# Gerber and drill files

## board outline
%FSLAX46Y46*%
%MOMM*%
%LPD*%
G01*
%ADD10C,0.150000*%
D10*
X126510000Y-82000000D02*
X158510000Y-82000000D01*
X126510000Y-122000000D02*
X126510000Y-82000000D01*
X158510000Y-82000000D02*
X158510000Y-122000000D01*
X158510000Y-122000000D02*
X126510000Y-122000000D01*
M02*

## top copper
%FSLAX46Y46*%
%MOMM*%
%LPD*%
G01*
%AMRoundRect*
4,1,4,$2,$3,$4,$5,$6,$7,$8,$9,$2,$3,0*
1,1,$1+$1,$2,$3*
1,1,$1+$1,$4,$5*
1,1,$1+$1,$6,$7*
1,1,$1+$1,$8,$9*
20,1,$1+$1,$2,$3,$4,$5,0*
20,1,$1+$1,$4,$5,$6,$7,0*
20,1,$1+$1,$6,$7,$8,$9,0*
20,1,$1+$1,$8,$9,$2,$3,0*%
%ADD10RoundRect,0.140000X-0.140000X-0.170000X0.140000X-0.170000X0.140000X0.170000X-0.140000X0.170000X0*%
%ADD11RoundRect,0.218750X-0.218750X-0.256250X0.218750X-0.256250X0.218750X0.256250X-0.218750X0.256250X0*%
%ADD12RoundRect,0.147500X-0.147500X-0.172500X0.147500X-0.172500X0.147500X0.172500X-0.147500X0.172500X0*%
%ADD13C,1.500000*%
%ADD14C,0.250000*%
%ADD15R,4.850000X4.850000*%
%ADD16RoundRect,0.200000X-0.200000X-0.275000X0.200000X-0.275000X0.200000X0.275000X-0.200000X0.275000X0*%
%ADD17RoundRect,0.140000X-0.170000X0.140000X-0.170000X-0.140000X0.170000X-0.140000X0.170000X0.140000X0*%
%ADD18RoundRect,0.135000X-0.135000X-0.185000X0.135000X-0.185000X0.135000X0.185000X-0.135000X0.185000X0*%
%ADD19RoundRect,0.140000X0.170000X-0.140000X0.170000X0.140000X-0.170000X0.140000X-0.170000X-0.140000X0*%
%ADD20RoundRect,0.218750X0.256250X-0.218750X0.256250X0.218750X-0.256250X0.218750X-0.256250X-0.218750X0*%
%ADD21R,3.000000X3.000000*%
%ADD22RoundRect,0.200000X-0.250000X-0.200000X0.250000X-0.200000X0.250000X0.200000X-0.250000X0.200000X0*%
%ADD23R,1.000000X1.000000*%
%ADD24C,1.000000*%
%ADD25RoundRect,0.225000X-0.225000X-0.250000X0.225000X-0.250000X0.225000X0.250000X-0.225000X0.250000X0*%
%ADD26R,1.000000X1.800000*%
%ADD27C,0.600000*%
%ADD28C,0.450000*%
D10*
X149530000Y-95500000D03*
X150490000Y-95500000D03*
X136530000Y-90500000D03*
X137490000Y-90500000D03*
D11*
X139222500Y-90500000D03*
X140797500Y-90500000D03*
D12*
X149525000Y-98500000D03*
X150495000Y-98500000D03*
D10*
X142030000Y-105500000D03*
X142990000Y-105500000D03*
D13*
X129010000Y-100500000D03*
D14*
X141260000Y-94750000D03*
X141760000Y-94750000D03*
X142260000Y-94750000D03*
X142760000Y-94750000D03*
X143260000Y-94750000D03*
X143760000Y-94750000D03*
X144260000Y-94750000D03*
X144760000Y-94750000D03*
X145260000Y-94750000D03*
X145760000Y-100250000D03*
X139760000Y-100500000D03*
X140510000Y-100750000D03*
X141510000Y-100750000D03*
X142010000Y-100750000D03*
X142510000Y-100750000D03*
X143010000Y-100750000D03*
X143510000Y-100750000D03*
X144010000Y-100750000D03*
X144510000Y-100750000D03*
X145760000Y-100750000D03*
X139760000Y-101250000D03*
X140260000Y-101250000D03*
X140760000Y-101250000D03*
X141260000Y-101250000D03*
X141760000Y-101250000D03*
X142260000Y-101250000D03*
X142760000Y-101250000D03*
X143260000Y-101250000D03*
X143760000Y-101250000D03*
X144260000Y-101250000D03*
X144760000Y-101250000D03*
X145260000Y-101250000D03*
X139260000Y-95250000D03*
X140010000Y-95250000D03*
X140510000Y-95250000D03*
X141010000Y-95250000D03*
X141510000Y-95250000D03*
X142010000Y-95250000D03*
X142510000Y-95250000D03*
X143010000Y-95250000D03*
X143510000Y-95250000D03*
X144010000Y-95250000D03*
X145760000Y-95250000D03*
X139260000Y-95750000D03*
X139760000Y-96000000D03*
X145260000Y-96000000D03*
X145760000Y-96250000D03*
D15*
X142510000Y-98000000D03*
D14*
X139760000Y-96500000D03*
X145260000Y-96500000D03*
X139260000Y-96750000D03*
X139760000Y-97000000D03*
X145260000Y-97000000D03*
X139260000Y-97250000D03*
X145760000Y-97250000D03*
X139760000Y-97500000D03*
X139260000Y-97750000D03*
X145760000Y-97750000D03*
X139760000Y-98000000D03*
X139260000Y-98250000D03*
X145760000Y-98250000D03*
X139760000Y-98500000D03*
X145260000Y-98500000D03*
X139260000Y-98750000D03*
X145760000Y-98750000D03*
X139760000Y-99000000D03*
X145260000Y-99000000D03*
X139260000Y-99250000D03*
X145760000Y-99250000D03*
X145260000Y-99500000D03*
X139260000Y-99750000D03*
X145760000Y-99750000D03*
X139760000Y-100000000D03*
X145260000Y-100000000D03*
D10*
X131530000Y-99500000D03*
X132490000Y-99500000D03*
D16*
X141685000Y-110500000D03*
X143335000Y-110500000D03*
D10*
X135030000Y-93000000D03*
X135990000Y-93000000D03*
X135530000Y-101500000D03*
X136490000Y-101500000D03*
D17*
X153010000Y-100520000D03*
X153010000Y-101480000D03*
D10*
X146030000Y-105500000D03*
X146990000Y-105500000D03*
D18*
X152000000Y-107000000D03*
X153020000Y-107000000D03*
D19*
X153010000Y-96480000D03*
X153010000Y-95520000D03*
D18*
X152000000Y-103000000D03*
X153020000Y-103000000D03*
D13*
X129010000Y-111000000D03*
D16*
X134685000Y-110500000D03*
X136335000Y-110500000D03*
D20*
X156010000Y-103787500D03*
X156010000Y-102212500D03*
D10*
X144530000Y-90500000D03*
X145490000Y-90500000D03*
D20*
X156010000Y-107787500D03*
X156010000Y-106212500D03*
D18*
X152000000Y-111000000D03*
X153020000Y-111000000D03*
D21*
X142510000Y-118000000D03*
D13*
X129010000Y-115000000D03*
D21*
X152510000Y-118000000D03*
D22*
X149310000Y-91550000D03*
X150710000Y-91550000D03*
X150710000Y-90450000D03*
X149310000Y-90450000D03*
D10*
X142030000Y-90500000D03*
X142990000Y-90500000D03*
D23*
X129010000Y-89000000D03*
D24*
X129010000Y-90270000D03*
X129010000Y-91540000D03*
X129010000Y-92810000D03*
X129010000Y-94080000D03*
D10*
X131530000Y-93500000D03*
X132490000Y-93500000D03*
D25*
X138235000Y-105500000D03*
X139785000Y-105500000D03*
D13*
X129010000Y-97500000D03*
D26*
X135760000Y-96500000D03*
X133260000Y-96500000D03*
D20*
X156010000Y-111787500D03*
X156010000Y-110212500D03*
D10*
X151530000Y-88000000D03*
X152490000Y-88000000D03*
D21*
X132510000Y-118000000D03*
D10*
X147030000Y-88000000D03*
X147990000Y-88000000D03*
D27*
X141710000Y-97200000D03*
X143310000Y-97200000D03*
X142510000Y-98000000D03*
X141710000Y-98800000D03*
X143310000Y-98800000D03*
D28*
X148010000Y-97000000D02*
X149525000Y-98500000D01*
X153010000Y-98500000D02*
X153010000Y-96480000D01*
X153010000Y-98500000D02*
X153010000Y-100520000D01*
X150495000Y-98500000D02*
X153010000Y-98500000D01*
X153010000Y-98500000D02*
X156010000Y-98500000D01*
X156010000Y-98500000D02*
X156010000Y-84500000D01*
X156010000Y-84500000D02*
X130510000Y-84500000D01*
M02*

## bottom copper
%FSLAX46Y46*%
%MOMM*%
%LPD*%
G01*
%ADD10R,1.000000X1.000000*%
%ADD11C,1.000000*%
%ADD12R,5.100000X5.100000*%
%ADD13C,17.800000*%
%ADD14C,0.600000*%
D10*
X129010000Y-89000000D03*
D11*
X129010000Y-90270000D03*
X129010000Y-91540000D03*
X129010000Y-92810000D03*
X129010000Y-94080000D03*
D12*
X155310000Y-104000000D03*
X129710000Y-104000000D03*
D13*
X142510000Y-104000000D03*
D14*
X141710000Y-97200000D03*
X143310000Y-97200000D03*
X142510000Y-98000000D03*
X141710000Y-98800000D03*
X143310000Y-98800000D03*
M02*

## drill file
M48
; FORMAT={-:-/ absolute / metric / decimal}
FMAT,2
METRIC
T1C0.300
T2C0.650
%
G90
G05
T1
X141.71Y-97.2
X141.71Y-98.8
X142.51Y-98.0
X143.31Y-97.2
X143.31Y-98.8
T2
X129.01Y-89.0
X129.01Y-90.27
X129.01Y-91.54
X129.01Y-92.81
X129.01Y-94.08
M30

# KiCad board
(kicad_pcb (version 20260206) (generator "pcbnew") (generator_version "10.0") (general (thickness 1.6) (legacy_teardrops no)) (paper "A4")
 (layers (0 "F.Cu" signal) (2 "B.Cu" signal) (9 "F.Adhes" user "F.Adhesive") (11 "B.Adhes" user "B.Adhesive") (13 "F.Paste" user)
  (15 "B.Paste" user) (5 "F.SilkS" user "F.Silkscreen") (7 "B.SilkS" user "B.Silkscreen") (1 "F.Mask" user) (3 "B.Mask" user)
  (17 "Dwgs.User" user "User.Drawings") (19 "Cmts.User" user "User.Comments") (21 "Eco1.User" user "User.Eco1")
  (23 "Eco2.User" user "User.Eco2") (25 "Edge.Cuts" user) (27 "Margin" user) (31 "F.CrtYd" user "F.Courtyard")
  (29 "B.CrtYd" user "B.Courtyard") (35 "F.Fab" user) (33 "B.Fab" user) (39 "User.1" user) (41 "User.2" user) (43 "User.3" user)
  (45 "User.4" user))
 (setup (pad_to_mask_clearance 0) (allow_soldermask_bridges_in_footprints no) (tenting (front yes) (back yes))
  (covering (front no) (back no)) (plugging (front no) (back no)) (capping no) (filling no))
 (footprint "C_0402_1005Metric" (layer "F.Cu") (at 150.01 95.5)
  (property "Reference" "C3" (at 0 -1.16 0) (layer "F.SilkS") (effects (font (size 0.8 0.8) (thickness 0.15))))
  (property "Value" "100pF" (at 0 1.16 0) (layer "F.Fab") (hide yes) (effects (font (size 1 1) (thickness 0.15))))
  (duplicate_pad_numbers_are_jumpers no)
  (pad "1" smd roundrect (at -0.48 0) (size 0.56 0.62) (layers "F.Cu" "F.Mask" "F.Paste") (roundrect_rratio 0.25) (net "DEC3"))
  (pad "2" smd roundrect (at 0.48 0) (size 0.56 0.62) (layers "F.Cu" "F.Mask" "F.Paste") (roundrect_rratio 0.25) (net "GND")))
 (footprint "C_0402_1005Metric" (layer "F.Cu") (at 137.01 90.5)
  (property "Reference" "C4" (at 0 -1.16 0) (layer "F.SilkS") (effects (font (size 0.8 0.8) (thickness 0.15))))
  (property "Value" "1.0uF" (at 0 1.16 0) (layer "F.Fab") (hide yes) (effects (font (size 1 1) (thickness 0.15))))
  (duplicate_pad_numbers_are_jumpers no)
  (pad "1" smd roundrect (at -0.48 0) (size 0.56 0.62) (layers "F.Cu" "F.Mask" "F.Paste") (roundrect_rratio 0.25) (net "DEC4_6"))
  (pad "2" smd roundrect (at 0.48 0) (size 0.56 0.62) (layers "F.Cu" "F.Mask" "F.Paste") (roundrect_rratio 0.25) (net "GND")))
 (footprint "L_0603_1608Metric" (layer "F.Cu") (at 140.01 90.5)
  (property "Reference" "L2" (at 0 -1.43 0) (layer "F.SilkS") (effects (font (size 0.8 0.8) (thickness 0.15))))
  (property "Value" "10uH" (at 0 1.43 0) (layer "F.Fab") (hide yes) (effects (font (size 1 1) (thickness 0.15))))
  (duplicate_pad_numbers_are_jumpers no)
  (pad "1" smd roundrect (at -0.7875 0) (size 0.875 0.95) (layers "F.Cu" "F.Mask" "F.Paste") (roundrect_rratio 0.25) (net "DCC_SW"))
  (pad "2" smd roundrect (at 0.7875 0) (size 0.875 0.95) (layers "F.Cu" "F.Mask" "F.Paste") (roundrect_rratio 0.25) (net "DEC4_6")))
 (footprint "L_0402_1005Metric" (layer "F.Cu") (at 150.01 98.5)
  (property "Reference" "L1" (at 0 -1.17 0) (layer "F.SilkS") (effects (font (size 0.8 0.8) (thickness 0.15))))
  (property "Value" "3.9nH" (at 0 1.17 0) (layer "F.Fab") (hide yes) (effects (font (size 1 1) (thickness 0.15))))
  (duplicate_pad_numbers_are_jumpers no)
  (pad "1" smd roundrect (at -0.485 0) (size 0.59 0.64) (layers "F.Cu" "F.Mask" "F.Paste") (roundrect_rratio 0.25) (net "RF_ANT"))
  (pad "2" smd roundrect (at 0.485 0) (size 0.59 0.64) (layers "F.Cu" "F.Mask" "F.Paste") (roundrect_rratio 0.25) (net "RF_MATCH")))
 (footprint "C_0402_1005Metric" (layer "F.Cu") (at 142.51 105.5)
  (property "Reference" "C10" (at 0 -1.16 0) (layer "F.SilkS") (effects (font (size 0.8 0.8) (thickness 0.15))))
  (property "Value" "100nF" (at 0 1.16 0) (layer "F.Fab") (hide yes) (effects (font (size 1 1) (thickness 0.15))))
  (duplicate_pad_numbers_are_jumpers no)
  (pad "1" smd roundrect (at -0.48 0) (size 0.56 0.62) (layers "F.Cu" "F.Mask" "F.Paste") (roundrect_rratio 0.25) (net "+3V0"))
  (pad "2" smd roundrect (at 0.48 0) (size 0.56 0.62) (layers "F.Cu" "F.Mask" "F.Paste") (roundrect_rratio 0.25) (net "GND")))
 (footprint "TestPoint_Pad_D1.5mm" (layer "F.Cu") (at 129.01 100.5)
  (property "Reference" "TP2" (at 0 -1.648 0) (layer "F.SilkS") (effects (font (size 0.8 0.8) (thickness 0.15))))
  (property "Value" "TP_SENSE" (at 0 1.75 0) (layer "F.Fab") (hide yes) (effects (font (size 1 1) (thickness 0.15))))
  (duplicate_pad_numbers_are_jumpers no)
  (pad "1" smd circle (at 0 0) (size 1.5 1.5) (layers "F.Cu" "F.Mask") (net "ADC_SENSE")))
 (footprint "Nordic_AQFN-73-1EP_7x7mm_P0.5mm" (layer "F.Cu") (at 142.51 98)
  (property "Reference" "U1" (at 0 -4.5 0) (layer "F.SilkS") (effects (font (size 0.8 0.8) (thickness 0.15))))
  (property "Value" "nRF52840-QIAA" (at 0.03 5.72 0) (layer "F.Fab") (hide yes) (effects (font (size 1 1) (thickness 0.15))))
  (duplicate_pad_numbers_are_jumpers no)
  (pad "" smd rect (at -1.2125 -1.2125 180) (size 2 2) (layers "F.Paste"))
  (pad "" smd rect (at -1.2125 1.2125 180) (size 2 2) (layers "F.Paste"))
  (pad "" smd rect (at 1.2125 -1.2125 180) (size 2 2) (layers "F.Paste"))
  (pad "" smd rect (at 1.2125 1.2125 180) (size 2 2) (layers "F.Paste"))
  (pad "A8" smd circle (at -1.25 -3.25 180) (size 0.25 0.25) (layers "F.Cu" "F.Mask" "F.Paste"))
  (pad "A10" smd circle (at -0.75 -3.25 180) (size 0.25 0.25) (layers "F.Cu" "F.Mask" "F.Paste"))
  (pad "A12" smd circle (at -0.25 -3.25 180) (size 0.25 0.25) (layers "F.Cu" "F.Mask" "F.Paste") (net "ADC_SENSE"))
  (pad "A14" smd circle (at 0.25 -3.25 180) (size 0.25 0.25) (layers "F.Cu" "F.Mask" "F.Paste"))
  (pad "A16" smd circle (at 0.75 -3.25 180) (size 0.25 0.25) (layers "F.Cu" "F.Mask" "F.Paste"))
  (pad "A18" smd circle (at 1.25 -3.25 180) (size 0.25 0.25) (layers "F.Cu" "F.Mask" "F.Paste"))
  (pad "A20" smd circle (at 1.75 -3.25 180) (size 0.25 0.25) (layers "F.Cu" "F.Mask" "F.Paste"))
  (pad "A22" smd circle (at 2.25 -3.25 180) (size 0.25 0.25) (layers "F.Cu" "F.Mask" "F.Paste") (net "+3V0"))
  (pad "A23" smd circle (at 2.75 -3.25 180) (size 0.25 0.25) (layers "F.Cu" "F.Mask" "F.Paste") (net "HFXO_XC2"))
  (pad "AA24" smd circle (at 3.25 2.25 180) (size 0.25 0.25) (layers "F.Cu" "F.Mask" "F.Paste") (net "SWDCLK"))
  (pad "AB2" smd circle (at -2.75 2.5 180) (size 0.25 0.25) (layers "F.Cu" "F.Mask" "F.Paste"))
  (pad "AC5" smd circle (at -2 2.75 180) (size 0.25 0.25) (layers "F.Cu" "F.Mask" "F.Paste"))
  (pad "AC9" smd circle (at -1 2.75 180) (size 0.25 0.25) (layers "F.Cu" "F.Mask" "F.Paste") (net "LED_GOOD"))
  (pad "AC11" smd circle (at -0.5 2.75 180) (size 0.25 0.25) (layers "F.Cu" "F.Mask" "F.Paste") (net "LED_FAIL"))
  (pad "AC13" smd circle (at 0 2.75 180) (size 0.25 0.25) (layers "F.Cu" "F.Mask" "F.Paste") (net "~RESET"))
  (pad "AC15" smd circle (at 0.5 2.75 180) (size 0.25 0.25) (layers "F.Cu" "F.Mask" "F.Paste"))
  (pad "AC17" smd circle (at 1 2.75 180) (size 0.25 0.25) (layers "F.Cu" "F.Mask" "F.Paste"))
  (pad "AC19" smd circle (at 1.5 2.75 180) (size 0.25 0.25) (layers "F.Cu" "F.Mask" "F.Paste"))
  (pad "AC21" smd circle (at 2 2.75 180) (size 0.25 0.25) (layers "F.Cu" "F.Mask" "F.Paste"))
  (pad "AC24" smd circle (at 3.25 2.75 180) (size 0.25 0.25) (layers "F.Cu" "F.Mask" "F.Paste") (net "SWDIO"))
  (pad "AD2" smd circle (at -2.75 3.25 180) (size 0.25 0.25) (layers "F.Cu" "F.Mask" "F.Paste") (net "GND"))
  (pad "AD4" smd circle (at -2.25 3.25 180) (size 0.25 0.25) (layers "F.Cu" "F.Mask" "F.Paste"))
  (pad "AD6" smd circle (at -1.75 3.25 180) (size 0.25 0.25) (layers "F.Cu" "F.Mask" "F.Paste"))
  (pad "AD8" smd circle (at -1.25 3.25 180) (size 0.25 0.25) (layers "F.Cu" "F.Mask" "F.Paste") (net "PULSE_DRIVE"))
  (pad "AD10" smd circle (at -0.75 3.25 180) (size 0.25 0.25) (layers "F.Cu" "F.Mask" "F.Paste") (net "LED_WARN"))
  (pad "AD12" smd circle (at -0.25 3.25 180) (size 0.25 0.25) (layers "F.Cu" "F.Mask" "F.Paste"))
  (pad "AD14" smd circle (at 0.25 3.25 180) (size 0.25 0.25) (layers "F.Cu" "F.Mask" "F.Paste") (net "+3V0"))
  (pad "AD16" smd circle (at 0.75 3.25 180) (size 0.25 0.25) (layers "F.Cu" "F.Mask" "F.Paste"))
  (pad "AD18" smd circle (at 1.25 3.25 180) (size 0.25 0.25) (layers "F.Cu" "F.Mask" "F.Paste"))
  (pad "AD20" smd circle (at 1.75 3.25 180) (size 0.25 0.25) (layers "F.Cu" "F.Mask" "F.Paste"))
  (pad "AD22" smd circle (at 2.25 3.25 180) (size 0.25 0.25) (layers "F.Cu" "F.Mask" "F.Paste"))
  (pad "AD23" smd circle (at 2.75 3.25 180) (size 0.25 0.25) (layers "F.Cu" "F.Mask" "F.Paste") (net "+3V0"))
  (pad "B1" smd circle (at -3.25 -2.75 180) (size 0.25 0.25) (layers "F.Cu" "F.Mask" "F.Paste") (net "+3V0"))
  (pad "B3" smd circle (at -2.5 -2.75 180) (size 0.25 0.25) (layers "F.Cu" "F.Mask" "F.Paste") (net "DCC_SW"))
  (pad "B5" smd circle (at -2 -2.75 180) (size 0.25 0.25) (layers "F.Cu" "F.Mask" "F.Paste") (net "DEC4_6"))
  (pad "B7" smd circle (at -1.5 -2.75 180) (size 0.25 0.25) (layers "F.Cu" "F.Mask" "F.Paste") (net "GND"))
  (pad "B9" smd circle (at -1 -2.75 180) (size 0.25 0.25) (layers "F.Cu" "F.Mask" "F.Paste"))
  (pad "B11" smd circle (at -0.5 -2.75 180) (size 0.25 0.25) (layers "F.Cu" "F.Mask" "F.Paste"))
  (pad "B13" smd circle (at 0 -2.75 180) (size 0.25 0.25) (layers "F.Cu" "F.Mask" "F.Paste"))
  (pad "B15" smd circle (at 0.5 -2.75 180) (size 0.25 0.25) (layers "F.Cu" "F.Mask" "F.Paste"))
  (pad "B17" smd circle (at 1 -2.75 180) (size 0.25 0.25) (layers "F.Cu" "F.Mask" "F.Paste"))
  (pad "B19" smd circle (at 1.5 -2.75 180) (size 0.25 0.25) (layers "F.Cu" "F.Mask" "F.Paste"))
  (pad "B24" smd circle (at 3.25 -2.75 180) (size 0.25 0.25) (layers "F.Cu" "F.Mask" "F.Paste") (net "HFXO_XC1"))
  (pad "C1" smd circle (at -3.25 -2.25 180) (size 0.25 0.25) (layers "F.Cu" "F.Mask" "F.Paste") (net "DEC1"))
  (pad "D2" smd circle (at -2.75 -2 180) (size 0.25 0.25) (layers "F.Cu" "F.Mask" "F.Paste") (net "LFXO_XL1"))
  (pad "D23" smd circle (at 2.75 -2 180) (size 0.25 0.25) (layers "F.Cu" "F.Mask" "F.Paste") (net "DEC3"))
  (pad "E24" smd circle (at 3.25 -1.75 180) (size 0.25 0.25) (layers "F.Cu" "F.Mask" "F.Paste") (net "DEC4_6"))
  (pad "EP" smd rect (at 0 0 180) (size 4.85 4.85) (layers "F.Cu" "F.Mask") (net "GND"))
  (pad "F2" smd circle (at -2.75 -1.5 180) (size 0.25 0.25) (layers "F.Cu" "F.Mask" "F.Paste") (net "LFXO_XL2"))
  (pad "F23" smd circle (at 2.75 -1.5 180) (size 0.25 0.25) (layers "F.Cu" "F.Mask" "F.Paste") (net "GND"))
  (pad "G1" smd circle (at -3.25 -1.25 180) (size 0.25 0.25) (layers "F.Cu" "F.Mask" "F.Paste"))
  (pad "H2" smd circle (at -2.75 -1 180) (size 0.25 0.25) (layers "F.Cu" "F.Mask" "F.Paste"))
  (pad "H23" smd circle (at 2.75 -1 180) (size 0.25 0.25) (layers "F.Cu" "F.Mask" "F.Paste") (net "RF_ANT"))
  (pad "J1" smd circle (at -3.25 -0.75 180) (size 0.25 0.25) (layers "F.Cu" "F.Mask" "F.Paste"))
  (pad "J24" smd circle (at 3.25 -0.75 180) (size 0.25 0.25) (layers "F.Cu" "F.Mask" "F.Paste"))
  (pad "K2" smd circle (at -2.75 -0.5 180) (size 0.25 0.25) (layers "F.Cu" "F.Mask" "F.Paste"))
  (pad "L1" smd circle (at -3.25 -0.25 180) (size 0.25 0.25) (layers "F.Cu" "F.Mask" "F.Paste"))
  (pad "L24" smd circle (at 3.25 -0.25 180) (size 0.25 0.25) (layers "F.Cu" "F.Mask" "F.Paste"))
  (pad "M2" smd circle (at -2.75 0 180) (size 0.25 0.25) (layers "F.Cu" "F.Mask" "F.Paste"))
  (pad "N1" smd circle (at -3.25 0.25 180) (size 0.25 0.25) (layers "F.Cu" "F.Mask" "F.Paste"))
  (pad "N24" smd circle (at 3.25 0.25 180) (size 0.25 0.25) (layers "F.Cu" "F.Mask" "F.Paste"))
  (pad "P2" smd circle (at -2.75 0.5 180) (size 0.25 0.25) (layers "F.Cu" "F.Mask" "F.Paste"))
  (pad "P23" smd circle (at 2.75 0.5 180) (size 0.25 0.25) (layers "F.Cu" "F.Mask" "F.Paste"))
  (pad "R1" smd circle (at -3.25 0.75 180) (size 0.25 0.25) (layers "F.Cu" "F.Mask" "F.Paste"))
  (pad "R24" smd circle (at 3.25 0.75 180) (size 0.25 0.25) (layers "F.Cu" "F.Mask" "F.Paste"))
  (pad "T2" smd circle (at -2.75 1 180) (size 0.25 0.25) (layers "F.Cu" "F.Mask" "F.Paste"))
  (pad "T23" smd circle (at 2.75 1 180) (size 0.25 0.25) (layers "F.Cu" "F.Mask" "F.Paste"))
  (pad "U1" smd circle (at -3.25 1.25 180) (size 0.25 0.25) (layers "F.Cu" "F.Mask" "F.Paste"))
  (pad "U24" smd circle (at 3.25 1.25 180) (size 0.25 0.25) (layers "F.Cu" "F.Mask" "F.Paste"))
  (pad "V23" smd circle (at 2.75 1.5 180) (size 0.25 0.25) (layers "F.Cu" "F.Mask" "F.Paste"))
  (pad "W1" smd circle (at -3.25 1.75 180) (size 0.25 0.25) (layers "F.Cu" "F.Mask" "F.Paste") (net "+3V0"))
  (pad "W24" smd circle (at 3.25 1.75 180) (size 0.25 0.25) (layers "F.Cu" "F.Mask" "F.Paste"))
  (pad "Y2" smd circle (at -2.75 2 180) (size 0.25 0.25) (layers "F.Cu" "F.Mask" "F.Paste") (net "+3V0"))
  (pad "Y23" smd circle (at 2.75 2 180) (size 0.25 0.25) (layers "F.Cu" "F.Mask" "F.Paste")))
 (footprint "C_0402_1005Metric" (layer "F.Cu") (at 132.01 99.5)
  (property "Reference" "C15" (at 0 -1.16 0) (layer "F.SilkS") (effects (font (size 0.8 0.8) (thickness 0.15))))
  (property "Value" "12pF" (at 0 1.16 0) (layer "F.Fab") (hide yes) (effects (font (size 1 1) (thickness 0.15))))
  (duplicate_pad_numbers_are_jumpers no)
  (pad "1" smd roundrect (at -0.48 0) (size 0.56 0.62) (layers "F.Cu" "F.Mask" "F.Paste") (roundrect_rratio 0.25) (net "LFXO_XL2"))
  (pad "2" smd roundrect (at 0.48 0) (size 0.56 0.62) (layers "F.Cu" "F.Mask" "F.Paste") (roundrect_rratio 0.25) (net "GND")))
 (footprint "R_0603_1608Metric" (layer "F.Cu") (at 142.51 110.5)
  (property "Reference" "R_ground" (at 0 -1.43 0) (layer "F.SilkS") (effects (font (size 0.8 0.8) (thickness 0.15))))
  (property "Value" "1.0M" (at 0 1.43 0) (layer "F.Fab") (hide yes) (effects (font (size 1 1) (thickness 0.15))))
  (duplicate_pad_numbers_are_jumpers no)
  (pad "1" smd roundrect (at -0.825 0) (size 0.8 0.95) (layers "F.Cu" "F.Mask" "F.Paste") (roundrect_rratio 0.25) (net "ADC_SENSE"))
  (pad "2" smd roundrect (at 0.825 0) (size 0.8 0.95) (layers "F.Cu" "F.Mask" "F.Paste") (roundrect_rratio 0.25) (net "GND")))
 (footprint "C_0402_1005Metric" (layer "F.Cu") (at 135.51 93)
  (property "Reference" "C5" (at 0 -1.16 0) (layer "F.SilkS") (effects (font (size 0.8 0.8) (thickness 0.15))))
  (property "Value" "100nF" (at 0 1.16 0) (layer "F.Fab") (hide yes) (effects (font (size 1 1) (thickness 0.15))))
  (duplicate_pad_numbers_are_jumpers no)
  (pad "1" smd roundrect (at -0.48 0) (size 0.56 0.62) (layers "F.Cu" "F.Mask" "F.Paste") (roundrect_rratio 0.25) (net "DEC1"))
  (pad "2" smd roundrect (at 0.48 0) (size 0.56 0.62) (layers "F.Cu" "F.Mask" "F.Paste") (roundrect_rratio 0.25) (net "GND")))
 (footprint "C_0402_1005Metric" (layer "F.Cu") (at 136.01 101.5)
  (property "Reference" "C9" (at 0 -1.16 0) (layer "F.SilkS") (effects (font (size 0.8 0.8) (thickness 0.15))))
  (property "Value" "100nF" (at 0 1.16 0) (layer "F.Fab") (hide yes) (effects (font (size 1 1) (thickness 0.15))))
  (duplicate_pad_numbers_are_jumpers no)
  (pad "1" smd roundrect (at -0.48 0) (size 0.56 0.62) (layers "F.Cu" "F.Mask" "F.Paste") (roundrect_rratio 0.25) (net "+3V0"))
  (pad "2" smd roundrect (at 0.48 0) (size 0.56 0.62) (layers "F.Cu" "F.Mask" "F.Paste") (roundrect_rratio 0.25) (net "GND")))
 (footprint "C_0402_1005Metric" (layer "F.Cu") (at 153.01 101 -90)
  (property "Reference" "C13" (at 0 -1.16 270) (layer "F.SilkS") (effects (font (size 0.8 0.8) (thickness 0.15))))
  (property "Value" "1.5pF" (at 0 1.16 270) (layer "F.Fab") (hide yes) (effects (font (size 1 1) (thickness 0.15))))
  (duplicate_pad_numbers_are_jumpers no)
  (pad "1" smd roundrect (at -0.48 0 270) (size 0.56 0.62) (layers "F.Cu" "F.Mask" "F.Paste") (roundrect_rratio 0.25) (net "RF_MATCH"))
  (pad "2" smd roundrect (at 0.48 0 270) (size 0.56 0.62) (layers "F.Cu" "F.Mask" "F.Paste") (roundrect_rratio 0.25) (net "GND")))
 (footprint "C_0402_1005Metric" (layer "F.Cu") (at 146.51 105.5)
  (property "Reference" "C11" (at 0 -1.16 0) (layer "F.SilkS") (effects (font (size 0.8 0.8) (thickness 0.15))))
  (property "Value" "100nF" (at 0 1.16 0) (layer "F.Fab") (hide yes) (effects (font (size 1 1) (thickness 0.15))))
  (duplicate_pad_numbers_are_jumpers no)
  (pad "1" smd roundrect (at -0.48 0) (size 0.56 0.62) (layers "F.Cu" "F.Mask" "F.Paste") (roundrect_rratio 0.25) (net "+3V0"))
  (pad "2" smd roundrect (at 0.48 0) (size 0.56 0.62) (layers "F.Cu" "F.Mask" "F.Paste") (roundrect_rratio 0.25) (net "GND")))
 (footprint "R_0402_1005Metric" (layer "F.Cu") (at 152.51 107)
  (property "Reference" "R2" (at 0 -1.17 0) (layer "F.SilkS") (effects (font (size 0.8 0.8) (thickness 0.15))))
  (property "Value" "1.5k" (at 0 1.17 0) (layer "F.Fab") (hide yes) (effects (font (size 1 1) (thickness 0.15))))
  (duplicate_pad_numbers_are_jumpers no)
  (pad "1" smd roundrect (at -0.51 0) (size 0.54 0.64) (layers "F.Cu" "F.Mask" "F.Paste") (roundrect_rratio 0.25) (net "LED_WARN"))
  (pad "2" smd roundrect (at 0.51 0) (size 0.54 0.64) (layers "F.Cu" "F.Mask" "F.Paste") (roundrect_rratio 0.25) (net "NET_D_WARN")))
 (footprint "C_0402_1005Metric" (layer "F.Cu") (at 153.01 96 90)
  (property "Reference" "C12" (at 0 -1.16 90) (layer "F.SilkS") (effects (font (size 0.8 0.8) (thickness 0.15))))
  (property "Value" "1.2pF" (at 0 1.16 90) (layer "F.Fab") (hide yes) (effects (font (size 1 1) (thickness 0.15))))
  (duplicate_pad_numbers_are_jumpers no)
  (pad "1" smd roundrect (at -0.48 0 90) (size 0.56 0.62) (layers "F.Cu" "F.Mask" "F.Paste") (roundrect_rratio 0.25) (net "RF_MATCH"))
  (pad "2" smd roundrect (at 0.48 0 90) (size 0.56 0.62) (layers "F.Cu" "F.Mask" "F.Paste") (roundrect_rratio 0.25) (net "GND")))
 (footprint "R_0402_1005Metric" (layer "F.Cu") (at 152.51 103)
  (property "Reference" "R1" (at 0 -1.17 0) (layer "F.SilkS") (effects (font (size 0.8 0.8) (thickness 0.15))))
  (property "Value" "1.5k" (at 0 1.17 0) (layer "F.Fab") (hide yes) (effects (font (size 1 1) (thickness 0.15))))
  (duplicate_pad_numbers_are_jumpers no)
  (pad "1" smd roundrect (at -0.51 0) (size 0.54 0.64) (layers "F.Cu" "F.Mask" "F.Paste") (roundrect_rratio 0.25) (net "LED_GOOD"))
  (pad "2" smd roundrect (at 0.51 0) (size 0.54 0.64) (layers "F.Cu" "F.Mask" "F.Paste") (roundrect_rratio 0.25) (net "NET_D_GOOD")))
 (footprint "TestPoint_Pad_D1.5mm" (layer "F.Cu") (at 129.01 111)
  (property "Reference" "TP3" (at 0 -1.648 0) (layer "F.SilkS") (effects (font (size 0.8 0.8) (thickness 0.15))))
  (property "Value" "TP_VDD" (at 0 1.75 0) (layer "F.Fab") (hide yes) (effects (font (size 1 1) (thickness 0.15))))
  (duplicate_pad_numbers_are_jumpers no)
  (pad "1" smd circle (at 0 0) (size 1.5 1.5) (layers "F.Cu" "F.Mask") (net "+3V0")))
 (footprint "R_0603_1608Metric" (layer "F.Cu") (at 135.51 110.5)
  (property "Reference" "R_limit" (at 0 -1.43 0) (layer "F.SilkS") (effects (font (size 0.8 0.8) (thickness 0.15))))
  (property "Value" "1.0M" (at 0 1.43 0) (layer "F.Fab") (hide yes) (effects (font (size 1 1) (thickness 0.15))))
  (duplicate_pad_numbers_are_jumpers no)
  (pad "1" smd roundrect (at -0.825 0) (size 0.8 0.95) (layers "F.Cu" "F.Mask" "F.Paste") (roundrect_rratio 0.25) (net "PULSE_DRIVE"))
  (pad "2" smd roundrect (at 0.825 0) (size 0.8 0.95) (layers "F.Cu" "F.Mask" "F.Paste") (roundrect_rratio 0.25) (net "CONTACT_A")))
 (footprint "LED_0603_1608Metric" (layer "F.Cu") (at 156.01 103 90)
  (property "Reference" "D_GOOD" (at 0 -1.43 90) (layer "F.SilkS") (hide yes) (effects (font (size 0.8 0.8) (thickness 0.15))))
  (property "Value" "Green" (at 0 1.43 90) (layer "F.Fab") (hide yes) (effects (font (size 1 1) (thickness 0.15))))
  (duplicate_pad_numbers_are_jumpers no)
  (pad "1" smd roundrect (at -0.7875 0 90) (size 0.875 0.95) (layers "F.Cu" "F.Mask" "F.Paste") (roundrect_rratio 0.25) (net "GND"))
  (pad "2" smd roundrect (at 0.7875 0 90) (size 0.875 0.95) (layers "F.Cu" "F.Mask" "F.Paste") (roundrect_rratio 0.25) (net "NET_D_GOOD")))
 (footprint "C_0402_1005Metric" (layer "F.Cu") (at 145.01 90.5)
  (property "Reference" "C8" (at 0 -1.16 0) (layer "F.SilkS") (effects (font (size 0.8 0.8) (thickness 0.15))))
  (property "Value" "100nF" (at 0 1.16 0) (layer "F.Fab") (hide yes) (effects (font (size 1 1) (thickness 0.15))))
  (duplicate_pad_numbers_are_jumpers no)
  (pad "1" smd roundrect (at -0.48 0) (size 0.56 0.62) (layers "F.Cu" "F.Mask" "F.Paste") (roundrect_rratio 0.25) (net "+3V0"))
  (pad "2" smd roundrect (at 0.48 0) (size 0.56 0.62) (layers "F.Cu" "F.Mask" "F.Paste") (roundrect_rratio 0.25) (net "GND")))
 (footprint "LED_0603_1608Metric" (layer "F.Cu") (at 156.01 107 90)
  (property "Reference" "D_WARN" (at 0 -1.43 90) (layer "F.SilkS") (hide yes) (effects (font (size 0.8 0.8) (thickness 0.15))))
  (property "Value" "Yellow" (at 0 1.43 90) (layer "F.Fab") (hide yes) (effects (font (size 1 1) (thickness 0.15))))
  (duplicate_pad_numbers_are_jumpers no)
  (pad "1" smd roundrect (at -0.7875 0 90) (size 0.875 0.95) (layers "F.Cu" "F.Mask" "F.Paste") (roundrect_rratio 0.25) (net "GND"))
  (pad "2" smd roundrect (at 0.7875 0 90) (size 0.875 0.95) (layers "F.Cu" "F.Mask" "F.Paste") (roundrect_rratio 0.25) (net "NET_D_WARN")))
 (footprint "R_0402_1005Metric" (layer "F.Cu") (at 152.51 111)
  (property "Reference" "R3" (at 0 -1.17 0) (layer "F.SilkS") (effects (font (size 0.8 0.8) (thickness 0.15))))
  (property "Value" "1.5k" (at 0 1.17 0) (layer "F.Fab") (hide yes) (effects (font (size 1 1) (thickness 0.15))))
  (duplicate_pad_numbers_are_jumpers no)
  (pad "1" smd roundrect (at -0.51 0) (size 0.54 0.64) (layers "F.Cu" "F.Mask" "F.Paste") (roundrect_rratio 0.25) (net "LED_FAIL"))
  (pad "2" smd roundrect (at 0.51 0) (size 0.54 0.64) (layers "F.Cu" "F.Mask" "F.Paste") (roundrect_rratio 0.25) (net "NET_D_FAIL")))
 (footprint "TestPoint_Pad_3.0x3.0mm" (layer "F.Cu") (at 142.51 118)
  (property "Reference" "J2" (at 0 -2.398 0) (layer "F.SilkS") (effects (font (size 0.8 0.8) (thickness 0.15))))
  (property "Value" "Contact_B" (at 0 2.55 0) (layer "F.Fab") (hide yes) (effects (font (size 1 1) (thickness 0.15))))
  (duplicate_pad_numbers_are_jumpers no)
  (pad "1" smd rect (at 0 0) (size 3 3) (layers "F.Cu" "F.Mask") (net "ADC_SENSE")))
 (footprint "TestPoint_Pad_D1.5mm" (layer "F.Cu") (at 129.01 115)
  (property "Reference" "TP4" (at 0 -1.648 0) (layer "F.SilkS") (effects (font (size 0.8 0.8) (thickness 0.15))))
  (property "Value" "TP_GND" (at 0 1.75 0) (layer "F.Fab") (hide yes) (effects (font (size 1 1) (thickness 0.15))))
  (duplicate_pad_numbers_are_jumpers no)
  (pad "1" smd circle (at 0 0) (size 1.5 1.5) (layers "F.Cu" "F.Mask") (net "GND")))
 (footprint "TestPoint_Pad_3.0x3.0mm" (layer "F.Cu") (at 152.51 118)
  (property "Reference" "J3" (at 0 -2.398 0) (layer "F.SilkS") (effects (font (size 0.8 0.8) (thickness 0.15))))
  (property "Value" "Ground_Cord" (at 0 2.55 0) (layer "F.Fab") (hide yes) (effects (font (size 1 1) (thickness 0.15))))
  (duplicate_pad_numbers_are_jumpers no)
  (pad "1" smd rect (at 0 0) (size 3 3) (layers "F.Cu" "F.Mask") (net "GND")))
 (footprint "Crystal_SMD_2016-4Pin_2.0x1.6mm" (layer "F.Cu") (at 150.01 91)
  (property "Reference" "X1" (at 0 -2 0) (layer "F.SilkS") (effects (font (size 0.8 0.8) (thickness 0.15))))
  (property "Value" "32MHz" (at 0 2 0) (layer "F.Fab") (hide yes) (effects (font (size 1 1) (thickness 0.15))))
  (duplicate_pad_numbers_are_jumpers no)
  (pad "1" smd roundrect (at -0.7 0.55) (size 0.9 0.8) (layers "F.Cu" "F.Mask" "F.Paste") (roundrect_rratio 0.25) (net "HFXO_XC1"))
  (pad "2" smd roundrect (at 0.7 0.55) (size 0.9 0.8) (layers "F.Cu" "F.Mask" "F.Paste") (roundrect_rratio 0.25) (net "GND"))
  (pad "3" smd roundrect (at 0.7 -0.55) (size 0.9 0.8) (layers "F.Cu" "F.Mask" "F.Paste") (roundrect_rratio 0.25) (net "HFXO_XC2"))
  (pad "4" smd roundrect (at -0.7 -0.55) (size 0.9 0.8) (layers "F.Cu" "F.Mask" "F.Paste") (roundrect_rratio 0.25) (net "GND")))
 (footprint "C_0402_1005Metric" (layer "F.Cu") (at 142.51 90.5)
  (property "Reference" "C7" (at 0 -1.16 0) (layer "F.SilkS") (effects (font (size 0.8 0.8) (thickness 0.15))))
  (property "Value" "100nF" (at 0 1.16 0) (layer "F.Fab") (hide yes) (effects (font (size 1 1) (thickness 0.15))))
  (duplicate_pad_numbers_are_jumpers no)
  (pad "1" smd roundrect (at -0.48 0) (size 0.56 0.62) (layers "F.Cu" "F.Mask" "F.Paste") (roundrect_rratio 0.25) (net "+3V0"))
  (pad "2" smd roundrect (at 0.48 0) (size 0.56 0.62) (layers "F.Cu" "F.Mask" "F.Paste") (roundrect_rratio 0.25) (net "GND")))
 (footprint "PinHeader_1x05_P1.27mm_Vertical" (layer "F.Cu") (at 129.01 89)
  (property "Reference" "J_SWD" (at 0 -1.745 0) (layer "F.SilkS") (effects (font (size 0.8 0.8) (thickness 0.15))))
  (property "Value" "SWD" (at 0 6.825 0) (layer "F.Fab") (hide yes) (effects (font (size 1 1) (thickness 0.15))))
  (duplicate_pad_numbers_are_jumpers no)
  (pad "1" thru_hole rect (at 0 0) (size 1 1) (drill 0.65) (layers "*.Cu" "*.Mask") (remove_unused_layers no) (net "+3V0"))
  (pad "2" thru_hole circle (at 0 1.27) (size 1 1) (drill 0.65) (layers "*.Cu" "*.Mask") (remove_unused_layers no) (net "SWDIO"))
  (pad "3" thru_hole circle (at 0 2.54) (size 1 1) (drill 0.65) (layers "*.Cu" "*.Mask") (remove_unused_layers no) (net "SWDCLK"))
  (pad "4" thru_hole circle (at 0 3.81) (size 1 1) (drill 0.65) (layers "*.Cu" "*.Mask") (remove_unused_layers no) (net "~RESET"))
  (pad "5" thru_hole circle (at 0 5.08) (size 1 1) (drill 0.65) (layers "*.Cu" "*.Mask") (remove_unused_layers no) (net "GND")))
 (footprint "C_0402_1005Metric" (layer "F.Cu") (at 132.01 93.5)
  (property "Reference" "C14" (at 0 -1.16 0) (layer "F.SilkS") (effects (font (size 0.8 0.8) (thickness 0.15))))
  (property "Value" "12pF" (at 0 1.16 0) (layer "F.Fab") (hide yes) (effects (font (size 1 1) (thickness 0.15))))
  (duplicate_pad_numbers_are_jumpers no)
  (pad "1" smd roundrect (at -0.48 0) (size 0.56 0.62) (layers "F.Cu" "F.Mask" "F.Paste") (roundrect_rratio 0.25) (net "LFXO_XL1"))
  (pad "2" smd roundrect (at 0.48 0) (size 0.56 0.62) (layers "F.Cu" "F.Mask" "F.Paste") (roundrect_rratio 0.25) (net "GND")))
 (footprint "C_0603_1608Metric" (layer "F.Cu") (at 139.01 105.5)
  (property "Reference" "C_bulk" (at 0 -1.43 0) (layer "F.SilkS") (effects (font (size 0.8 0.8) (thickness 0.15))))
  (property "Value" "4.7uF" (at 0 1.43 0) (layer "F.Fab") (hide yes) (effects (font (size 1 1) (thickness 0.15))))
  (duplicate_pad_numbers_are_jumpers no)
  (pad "1" smd roundrect (at -0.775 0) (size 0.9 0.95) (layers "F.Cu" "F.Mask" "F.Paste") (roundrect_rratio 0.25) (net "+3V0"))
  (pad "2" smd roundrect (at 0.775 0) (size 0.9 0.95) (layers "F.Cu" "F.Mask" "F.Paste") (roundrect_rratio 0.25) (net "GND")))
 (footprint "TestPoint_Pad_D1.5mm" (layer "F.Cu") (at 129.01 97.5)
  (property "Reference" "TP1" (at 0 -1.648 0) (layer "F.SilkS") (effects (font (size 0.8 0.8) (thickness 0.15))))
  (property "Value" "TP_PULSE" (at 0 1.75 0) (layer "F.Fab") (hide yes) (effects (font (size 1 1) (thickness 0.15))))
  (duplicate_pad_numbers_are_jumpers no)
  (pad "1" smd circle (at 0 0) (size 1.5 1.5) (layers "F.Cu" "F.Mask") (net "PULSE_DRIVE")))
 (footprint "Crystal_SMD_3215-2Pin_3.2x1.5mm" (layer "F.Cu") (at 134.51 96.5)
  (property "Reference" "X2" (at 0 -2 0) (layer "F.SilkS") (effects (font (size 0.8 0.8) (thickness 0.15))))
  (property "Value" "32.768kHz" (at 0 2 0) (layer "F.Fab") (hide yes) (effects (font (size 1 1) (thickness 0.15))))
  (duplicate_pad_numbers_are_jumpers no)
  (pad "1" smd rect (at 1.25 0) (size 1 1.8) (layers "F.Cu" "F.Mask" "F.Paste") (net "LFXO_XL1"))
  (pad "2" smd rect (at -1.25 0) (size 1 1.8) (layers "F.Cu" "F.Mask" "F.Paste") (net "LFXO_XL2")))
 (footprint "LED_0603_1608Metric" (layer "F.Cu") (at 156.01 111 90)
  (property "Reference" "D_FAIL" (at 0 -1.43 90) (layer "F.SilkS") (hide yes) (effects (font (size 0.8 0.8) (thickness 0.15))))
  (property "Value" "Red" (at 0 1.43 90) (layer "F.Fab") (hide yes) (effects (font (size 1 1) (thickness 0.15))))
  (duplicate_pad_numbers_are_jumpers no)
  (pad "1" smd roundrect (at -0.7875 0 90) (size 0.875 0.95) (layers "F.Cu" "F.Mask" "F.Paste") (roundrect_rratio 0.25) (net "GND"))
  (pad "2" smd roundrect (at 0.7875 0 90) (size 0.875 0.95) (layers "F.Cu" "F.Mask" "F.Paste") (roundrect_rratio 0.25) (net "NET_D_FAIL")))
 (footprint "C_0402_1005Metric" (layer "F.Cu") (at 152.01 88)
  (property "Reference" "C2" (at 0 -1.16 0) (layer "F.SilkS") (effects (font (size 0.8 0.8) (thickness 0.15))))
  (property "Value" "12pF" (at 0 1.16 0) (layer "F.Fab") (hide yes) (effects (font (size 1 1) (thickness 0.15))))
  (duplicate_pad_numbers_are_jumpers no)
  (pad "1" smd roundrect (at -0.48 0) (size 0.56 0.62) (layers "F.Cu" "F.Mask" "F.Paste") (roundrect_rratio 0.25) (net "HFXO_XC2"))
  (pad "2" smd roundrect (at 0.48 0) (size 0.56 0.62) (layers "F.Cu" "F.Mask" "F.Paste") (roundrect_rratio 0.25) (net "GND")))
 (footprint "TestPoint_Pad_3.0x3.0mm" (layer "F.Cu") (at 132.51 118)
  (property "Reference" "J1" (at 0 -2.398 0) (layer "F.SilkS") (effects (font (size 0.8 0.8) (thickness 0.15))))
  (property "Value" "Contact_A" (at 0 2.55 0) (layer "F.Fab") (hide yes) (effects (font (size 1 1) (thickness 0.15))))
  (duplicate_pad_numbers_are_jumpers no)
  (pad "1" smd rect (at 0 0) (size 3 3) (layers "F.Cu" "F.Mask") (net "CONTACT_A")))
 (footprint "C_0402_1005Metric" (layer "F.Cu") (at 147.51 88)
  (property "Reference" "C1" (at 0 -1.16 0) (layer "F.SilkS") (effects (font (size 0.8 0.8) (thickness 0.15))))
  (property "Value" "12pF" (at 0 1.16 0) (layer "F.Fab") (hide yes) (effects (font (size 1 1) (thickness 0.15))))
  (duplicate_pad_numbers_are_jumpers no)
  (pad "1" smd roundrect (at -0.48 0) (size 0.56 0.62) (layers "F.Cu" "F.Mask" "F.Paste") (roundrect_rratio 0.25) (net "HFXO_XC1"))
  (pad "2" smd roundrect (at 0.48 0) (size 0.56 0.62) (layers "F.Cu" "F.Mask" "F.Paste") (roundrect_rratio 0.25) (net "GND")))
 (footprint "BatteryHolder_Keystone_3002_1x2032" (layer "B.Cu") (at 142.51 104 180)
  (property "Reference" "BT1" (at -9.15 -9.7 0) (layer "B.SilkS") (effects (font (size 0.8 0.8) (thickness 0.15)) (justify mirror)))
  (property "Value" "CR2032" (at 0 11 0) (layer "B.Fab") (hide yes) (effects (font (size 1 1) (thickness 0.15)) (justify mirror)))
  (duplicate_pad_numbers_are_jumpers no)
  (pad "1" smd rect (at -12.8 0 180) (size 5.1 5.1) (layers "B.Cu" "B.Mask" "B.Paste") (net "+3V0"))
  (pad "1" smd rect (at 12.8 0 180) (size 5.1 5.1) (layers "B.Cu" "B.Mask" "B.Paste"))
  (pad "2" smd circle (at 0 0 180) (size 17.8 17.8) (layers "B.Cu" "B.Mask") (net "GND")))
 (gr_line (start 126.51 82) (end 158.51 82) (stroke (width 0.15) (type default)) (layer "Edge.Cuts"))
 (gr_line (start 126.51 122) (end 126.51 82) (stroke (width 0.15) (type default)) (layer "Edge.Cuts"))
 (gr_line (start 158.51 82) (end 158.51 122) (stroke (width 0.15) (type default)) (layer "Edge.Cuts"))
 (gr_line (start 158.51 122) (end 126.51 122) (stroke (width 0.15) (type default)) (layer "Edge.Cuts"))
 (via (at 141.71 97.2) (size 0.6) (drill 0.3) (layers "F.Cu" "B.Cu") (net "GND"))
 (via (at 143.31 97.2) (size 0.6) (drill 0.3) (layers "F.Cu" "B.Cu") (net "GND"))
 (via (at 142.51 98) (size 0.6) (drill 0.3) (layers "F.Cu" "B.Cu") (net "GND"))
 (via (at 141.71 98.8) (size 0.6) (drill 0.3) (layers "F.Cu" "B.Cu") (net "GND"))
 (via (at 143.31 98.8) (size 0.6) (drill 0.3) (layers "F.Cu" "B.Cu") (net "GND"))
 (segment (start 148.01 97) (end 149.525 98.5) (width 0.45) (layer "F.Cu") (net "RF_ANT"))
 (segment (start 153.01 98.5) (end 153.01 96.48) (width 0.45) (layer "F.Cu") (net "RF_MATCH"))
 (segment (start 153.01 98.5) (end 153.01 100.52) (width 0.45) (layer "F.Cu") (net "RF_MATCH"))
 (segment (start 150.495 98.5) (end 153.01 98.5) (width 0.45) (layer "F.Cu") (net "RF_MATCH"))
 (segment (start 153.01 98.5) (end 156.01 98.5) (width 0.45) (layer "F.Cu") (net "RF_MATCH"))
 (segment (start 156.01 98.5) (end 156.01 84.5) (width 0.45) (layer "F.Cu") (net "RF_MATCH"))
 (segment (start 156.01 84.5) (end 130.51 84.5) (width 0.45) (layer "F.Cu") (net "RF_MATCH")))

